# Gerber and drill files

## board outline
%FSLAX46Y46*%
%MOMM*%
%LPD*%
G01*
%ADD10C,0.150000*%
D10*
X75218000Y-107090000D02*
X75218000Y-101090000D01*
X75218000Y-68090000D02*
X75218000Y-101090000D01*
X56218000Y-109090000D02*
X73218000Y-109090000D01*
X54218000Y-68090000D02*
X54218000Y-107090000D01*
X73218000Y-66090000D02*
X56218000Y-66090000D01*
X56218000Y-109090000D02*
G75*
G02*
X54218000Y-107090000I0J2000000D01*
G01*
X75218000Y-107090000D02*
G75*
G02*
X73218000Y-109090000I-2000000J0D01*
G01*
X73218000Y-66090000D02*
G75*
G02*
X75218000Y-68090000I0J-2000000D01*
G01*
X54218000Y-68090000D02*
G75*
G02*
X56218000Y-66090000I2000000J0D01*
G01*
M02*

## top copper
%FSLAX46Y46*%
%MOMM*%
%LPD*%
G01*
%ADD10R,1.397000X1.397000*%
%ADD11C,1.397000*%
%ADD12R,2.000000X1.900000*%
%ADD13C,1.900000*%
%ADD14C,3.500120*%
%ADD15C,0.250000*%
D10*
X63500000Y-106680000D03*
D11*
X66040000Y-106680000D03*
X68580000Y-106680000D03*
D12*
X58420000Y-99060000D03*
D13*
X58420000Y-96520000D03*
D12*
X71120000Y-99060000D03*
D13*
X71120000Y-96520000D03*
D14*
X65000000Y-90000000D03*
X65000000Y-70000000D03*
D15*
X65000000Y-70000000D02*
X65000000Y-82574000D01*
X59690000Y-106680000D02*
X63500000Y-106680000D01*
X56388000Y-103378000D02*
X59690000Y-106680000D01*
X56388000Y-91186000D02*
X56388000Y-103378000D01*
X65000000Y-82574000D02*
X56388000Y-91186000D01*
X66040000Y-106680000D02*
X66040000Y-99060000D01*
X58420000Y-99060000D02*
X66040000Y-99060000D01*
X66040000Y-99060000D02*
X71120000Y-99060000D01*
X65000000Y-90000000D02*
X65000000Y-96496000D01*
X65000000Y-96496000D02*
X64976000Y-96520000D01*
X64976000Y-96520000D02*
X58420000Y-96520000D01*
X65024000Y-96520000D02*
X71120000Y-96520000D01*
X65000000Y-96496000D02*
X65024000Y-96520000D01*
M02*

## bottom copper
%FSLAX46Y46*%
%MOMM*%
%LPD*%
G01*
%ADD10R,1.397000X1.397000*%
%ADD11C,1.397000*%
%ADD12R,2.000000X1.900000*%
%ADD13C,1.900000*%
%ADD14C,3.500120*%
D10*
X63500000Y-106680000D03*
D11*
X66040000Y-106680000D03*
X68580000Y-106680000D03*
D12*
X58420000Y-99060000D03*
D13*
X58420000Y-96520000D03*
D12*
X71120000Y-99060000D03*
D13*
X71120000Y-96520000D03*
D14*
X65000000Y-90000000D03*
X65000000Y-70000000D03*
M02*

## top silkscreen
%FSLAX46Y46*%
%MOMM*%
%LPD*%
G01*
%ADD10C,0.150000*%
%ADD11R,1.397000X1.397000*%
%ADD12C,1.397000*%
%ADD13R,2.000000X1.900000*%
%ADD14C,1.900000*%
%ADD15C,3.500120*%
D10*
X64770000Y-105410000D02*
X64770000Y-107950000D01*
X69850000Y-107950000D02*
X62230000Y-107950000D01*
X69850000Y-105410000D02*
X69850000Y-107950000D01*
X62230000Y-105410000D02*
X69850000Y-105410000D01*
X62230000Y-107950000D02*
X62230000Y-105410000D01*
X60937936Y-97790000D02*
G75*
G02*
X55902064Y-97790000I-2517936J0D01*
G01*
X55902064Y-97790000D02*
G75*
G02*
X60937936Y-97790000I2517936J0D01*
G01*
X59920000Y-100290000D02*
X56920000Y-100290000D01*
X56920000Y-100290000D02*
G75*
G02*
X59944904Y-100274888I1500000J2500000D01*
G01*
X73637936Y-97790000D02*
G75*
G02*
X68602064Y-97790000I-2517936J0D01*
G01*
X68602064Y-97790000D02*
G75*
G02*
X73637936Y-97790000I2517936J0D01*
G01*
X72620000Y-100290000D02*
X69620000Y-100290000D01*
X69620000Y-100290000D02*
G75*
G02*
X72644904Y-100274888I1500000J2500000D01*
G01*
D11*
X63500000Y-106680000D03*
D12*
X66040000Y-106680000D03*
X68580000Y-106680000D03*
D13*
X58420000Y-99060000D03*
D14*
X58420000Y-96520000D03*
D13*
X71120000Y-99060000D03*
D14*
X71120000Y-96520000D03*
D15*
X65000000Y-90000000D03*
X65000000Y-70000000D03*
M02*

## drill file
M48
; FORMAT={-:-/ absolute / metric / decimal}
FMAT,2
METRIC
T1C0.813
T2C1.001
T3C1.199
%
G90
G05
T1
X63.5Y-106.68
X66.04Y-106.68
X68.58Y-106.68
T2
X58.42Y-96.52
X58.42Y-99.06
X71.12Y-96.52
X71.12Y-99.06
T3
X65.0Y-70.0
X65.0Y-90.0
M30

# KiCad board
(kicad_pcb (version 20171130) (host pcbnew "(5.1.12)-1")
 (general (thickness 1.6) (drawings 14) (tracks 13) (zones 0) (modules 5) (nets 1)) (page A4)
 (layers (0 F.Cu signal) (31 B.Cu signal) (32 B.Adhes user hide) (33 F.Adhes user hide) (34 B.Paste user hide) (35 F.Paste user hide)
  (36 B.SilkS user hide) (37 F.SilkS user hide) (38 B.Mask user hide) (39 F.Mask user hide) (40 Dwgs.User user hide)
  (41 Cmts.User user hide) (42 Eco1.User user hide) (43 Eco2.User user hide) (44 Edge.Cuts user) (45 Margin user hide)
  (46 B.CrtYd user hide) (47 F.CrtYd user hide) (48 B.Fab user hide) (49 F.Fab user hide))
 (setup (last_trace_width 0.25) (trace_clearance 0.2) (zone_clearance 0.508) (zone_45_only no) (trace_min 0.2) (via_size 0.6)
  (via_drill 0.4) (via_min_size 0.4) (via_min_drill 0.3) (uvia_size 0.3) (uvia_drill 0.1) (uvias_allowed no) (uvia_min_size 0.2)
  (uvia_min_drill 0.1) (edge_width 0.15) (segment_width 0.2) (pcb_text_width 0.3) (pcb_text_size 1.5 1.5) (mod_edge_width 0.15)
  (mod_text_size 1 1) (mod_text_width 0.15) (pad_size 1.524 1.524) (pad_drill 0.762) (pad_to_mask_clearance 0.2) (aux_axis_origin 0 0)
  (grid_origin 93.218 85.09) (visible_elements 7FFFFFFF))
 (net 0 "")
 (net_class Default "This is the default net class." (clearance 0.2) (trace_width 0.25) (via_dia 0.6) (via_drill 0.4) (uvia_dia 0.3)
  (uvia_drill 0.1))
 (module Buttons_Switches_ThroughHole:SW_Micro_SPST (layer F.Cu) (at 66.04 106.68)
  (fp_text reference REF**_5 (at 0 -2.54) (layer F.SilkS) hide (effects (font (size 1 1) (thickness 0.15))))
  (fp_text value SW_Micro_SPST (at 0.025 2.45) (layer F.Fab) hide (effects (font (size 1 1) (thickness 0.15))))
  (fp_line (start -1.27 -1.27) (end -1.27 1.27) (layer F.SilkS) (width 0.15))
  (fp_line (start 3.81 1.27) (end -3.81 1.27) (layer F.SilkS) (width 0.15))
  (fp_line (start 3.81 -1.27) (end 3.81 1.27) (layer F.SilkS) (width 0.15))
  (fp_line (start -3.81 -1.27) (end 3.81 -1.27) (layer F.SilkS) (width 0.15))
  (fp_line (start -3.81 1.27) (end -3.81 -1.27) (layer F.SilkS) (width 0.15))
  (pad 1 thru_hole rect (at -2.54 0) (size 1.397 1.397) (drill 0.8128) (layers *.Cu *.Mask F.SilkS))
  (pad 2 thru_hole circle (at 0 0) (size 1.397 1.397) (drill 0.8128) (layers *.Cu *.Mask F.SilkS))
  (pad 3 thru_hole circle (at 2.54 0) (size 1.397 1.397) (drill 0.8128) (layers *.Cu *.Mask F.SilkS)))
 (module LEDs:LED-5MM (layer F.Cu) (at 58.42 99.06 90)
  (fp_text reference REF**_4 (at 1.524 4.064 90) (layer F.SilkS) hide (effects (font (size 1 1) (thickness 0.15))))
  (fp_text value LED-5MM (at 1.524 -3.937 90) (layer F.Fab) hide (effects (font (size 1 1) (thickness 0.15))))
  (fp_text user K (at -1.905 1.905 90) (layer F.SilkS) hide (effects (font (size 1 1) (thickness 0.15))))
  (fp_circle (center 1.27 0) (end 0.97 -2.5) (layer F.SilkS) (width 0.15))
  (fp_line (start -1.23 1.5) (end -1.23 -1.5) (layer F.SilkS) (width 0.15))
  (fp_arc (start 1.27 0) (end -1.23 -1.5) (angle 297.5) (layer F.SilkS) (width 0.15))
  (pad 1 thru_hole rect (at 0 0 180) (size 2 1.9) (drill 1.00076) (layers *.Cu *.Mask F.SilkS))
  (pad 2 thru_hole circle (at 2.54 0 90) (size 1.9 1.9) (drill 1.00076) (layers *.Cu *.Mask F.SilkS)))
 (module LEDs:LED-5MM (layer F.Cu) (at 71.12 99.06 90)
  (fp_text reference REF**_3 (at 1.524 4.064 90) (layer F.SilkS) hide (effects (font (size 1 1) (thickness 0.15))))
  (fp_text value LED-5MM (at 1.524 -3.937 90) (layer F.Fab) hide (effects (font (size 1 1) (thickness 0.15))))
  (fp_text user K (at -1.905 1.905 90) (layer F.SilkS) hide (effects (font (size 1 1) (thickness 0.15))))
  (fp_circle (center 1.27 0) (end 0.97 -2.5) (layer F.SilkS) (width 0.15))
  (fp_line (start -1.23 1.5) (end -1.23 -1.5) (layer F.SilkS) (width 0.15))
  (fp_arc (start 1.27 0) (end -1.23 -1.5) (angle 297.5) (layer F.SilkS) (width 0.15))
  (pad 1 thru_hole rect (at 0 0 180) (size 2 1.9) (drill 1.00076) (layers *.Cu *.Mask F.SilkS))
  (pad 2 thru_hole circle (at 2.54 0 90) (size 1.9 1.9) (drill 1.00076) (layers *.Cu *.Mask F.SilkS)))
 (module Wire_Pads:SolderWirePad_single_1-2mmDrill (layer F.Cu) (at 65 90)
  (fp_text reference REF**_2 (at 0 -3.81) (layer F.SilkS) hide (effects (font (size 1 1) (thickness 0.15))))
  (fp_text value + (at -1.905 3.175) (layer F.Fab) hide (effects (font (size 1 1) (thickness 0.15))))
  (pad 1 thru_hole circle (at 0 0) (size 3.50012 3.50012) (drill 1.19888) (layers *.Cu *.Mask F.SilkS)))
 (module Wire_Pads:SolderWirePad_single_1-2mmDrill (layer F.Cu) (at 65 70)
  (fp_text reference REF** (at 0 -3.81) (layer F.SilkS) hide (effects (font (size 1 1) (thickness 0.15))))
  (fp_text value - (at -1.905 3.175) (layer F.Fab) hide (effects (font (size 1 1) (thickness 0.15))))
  (pad 1 thru_hole circle (at 0 0) (size 3.50012 3.50012) (drill 1.19888) (layers *.Cu *.Mask F.SilkS)))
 (gr_line (start 75.218 107.09) (end 75.218 101.09) (angle 90) (layer Edge.Cuts) (width 0.15))
 (gr_line (start 75.218 68.09) (end 75.218 101.09) (angle 90) (layer Edge.Cuts) (width 0.15))
 (gr_line (start 56.218 109.09) (end 73.218 109.09) (angle 90) (layer Edge.Cuts) (width 0.15))
 (gr_line (start 54.218 68.09) (end 54.218 107.09) (angle 90) (layer Edge.Cuts) (width 0.15))
 (gr_line (start 73.218 66.09) (end 56.218 66.09) (angle 90) (layer Edge.Cuts) (width 0.15))
 (gr_arc (start 56.218 107.09) (end 56.218 109.09) (angle 90) (layer Edge.Cuts) (width 0.15))
 (gr_arc (start 73.218 107.09) (end 75.218 107.09) (angle 90) (layer Edge.Cuts) (width 0.15))
 (gr_arc (start 73.218 68.09) (end 73.218 66.09) (angle 90) (layer Edge.Cuts) (width 0.15))
 (gr_arc (start 56.218 68.09) (end 54.218 68.09) (angle 90) (layer Edge.Cuts) (width 0.15))
 (segment (start 65 70) (end 65 82.574) (width 0.25) (layer F.Cu) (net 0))
 (segment (start 59.69 106.68) (end 63.5 106.68) (width 0.25) (layer F.Cu) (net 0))
 (segment (start 56.388 103.378) (end 59.69 106.68) (width 0.25) (layer F.Cu) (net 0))
 (segment (start 56.388 91.186) (end 56.388 103.378) (width 0.25) (layer F.Cu) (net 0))
 (segment (start 65 82.574) (end 56.388 91.186) (width 0.25) (layer F.Cu) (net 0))
 (segment (start 66.04 106.68) (end 66.04 99.06) (width 0.25) (layer F.Cu) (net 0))
 (segment (start 58.42 99.06) (end 66.04 99.06) (width 0.25) (layer F.Cu) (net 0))
 (segment (start 66.04 99.06) (end 71.12 99.06) (width 0.25) (layer F.Cu) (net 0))
 (segment (start 65 90) (end 65 96.496) (width 0.25) (layer F.Cu) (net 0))
 (segment (start 65 96.496) (end 64.976 96.52) (width 0.25) (layer F.Cu) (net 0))
 (segment (start 64.976 96.52) (end 58.42 96.52) (width 0.25) (layer F.Cu) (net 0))
 (segment (start 65.024 96.52) (end 71.12 96.52) (width 0.25) (layer F.Cu) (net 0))
 (segment (start 65 96.496) (end 65.024 96.52) (width 0.25) (layer F.Cu) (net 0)))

